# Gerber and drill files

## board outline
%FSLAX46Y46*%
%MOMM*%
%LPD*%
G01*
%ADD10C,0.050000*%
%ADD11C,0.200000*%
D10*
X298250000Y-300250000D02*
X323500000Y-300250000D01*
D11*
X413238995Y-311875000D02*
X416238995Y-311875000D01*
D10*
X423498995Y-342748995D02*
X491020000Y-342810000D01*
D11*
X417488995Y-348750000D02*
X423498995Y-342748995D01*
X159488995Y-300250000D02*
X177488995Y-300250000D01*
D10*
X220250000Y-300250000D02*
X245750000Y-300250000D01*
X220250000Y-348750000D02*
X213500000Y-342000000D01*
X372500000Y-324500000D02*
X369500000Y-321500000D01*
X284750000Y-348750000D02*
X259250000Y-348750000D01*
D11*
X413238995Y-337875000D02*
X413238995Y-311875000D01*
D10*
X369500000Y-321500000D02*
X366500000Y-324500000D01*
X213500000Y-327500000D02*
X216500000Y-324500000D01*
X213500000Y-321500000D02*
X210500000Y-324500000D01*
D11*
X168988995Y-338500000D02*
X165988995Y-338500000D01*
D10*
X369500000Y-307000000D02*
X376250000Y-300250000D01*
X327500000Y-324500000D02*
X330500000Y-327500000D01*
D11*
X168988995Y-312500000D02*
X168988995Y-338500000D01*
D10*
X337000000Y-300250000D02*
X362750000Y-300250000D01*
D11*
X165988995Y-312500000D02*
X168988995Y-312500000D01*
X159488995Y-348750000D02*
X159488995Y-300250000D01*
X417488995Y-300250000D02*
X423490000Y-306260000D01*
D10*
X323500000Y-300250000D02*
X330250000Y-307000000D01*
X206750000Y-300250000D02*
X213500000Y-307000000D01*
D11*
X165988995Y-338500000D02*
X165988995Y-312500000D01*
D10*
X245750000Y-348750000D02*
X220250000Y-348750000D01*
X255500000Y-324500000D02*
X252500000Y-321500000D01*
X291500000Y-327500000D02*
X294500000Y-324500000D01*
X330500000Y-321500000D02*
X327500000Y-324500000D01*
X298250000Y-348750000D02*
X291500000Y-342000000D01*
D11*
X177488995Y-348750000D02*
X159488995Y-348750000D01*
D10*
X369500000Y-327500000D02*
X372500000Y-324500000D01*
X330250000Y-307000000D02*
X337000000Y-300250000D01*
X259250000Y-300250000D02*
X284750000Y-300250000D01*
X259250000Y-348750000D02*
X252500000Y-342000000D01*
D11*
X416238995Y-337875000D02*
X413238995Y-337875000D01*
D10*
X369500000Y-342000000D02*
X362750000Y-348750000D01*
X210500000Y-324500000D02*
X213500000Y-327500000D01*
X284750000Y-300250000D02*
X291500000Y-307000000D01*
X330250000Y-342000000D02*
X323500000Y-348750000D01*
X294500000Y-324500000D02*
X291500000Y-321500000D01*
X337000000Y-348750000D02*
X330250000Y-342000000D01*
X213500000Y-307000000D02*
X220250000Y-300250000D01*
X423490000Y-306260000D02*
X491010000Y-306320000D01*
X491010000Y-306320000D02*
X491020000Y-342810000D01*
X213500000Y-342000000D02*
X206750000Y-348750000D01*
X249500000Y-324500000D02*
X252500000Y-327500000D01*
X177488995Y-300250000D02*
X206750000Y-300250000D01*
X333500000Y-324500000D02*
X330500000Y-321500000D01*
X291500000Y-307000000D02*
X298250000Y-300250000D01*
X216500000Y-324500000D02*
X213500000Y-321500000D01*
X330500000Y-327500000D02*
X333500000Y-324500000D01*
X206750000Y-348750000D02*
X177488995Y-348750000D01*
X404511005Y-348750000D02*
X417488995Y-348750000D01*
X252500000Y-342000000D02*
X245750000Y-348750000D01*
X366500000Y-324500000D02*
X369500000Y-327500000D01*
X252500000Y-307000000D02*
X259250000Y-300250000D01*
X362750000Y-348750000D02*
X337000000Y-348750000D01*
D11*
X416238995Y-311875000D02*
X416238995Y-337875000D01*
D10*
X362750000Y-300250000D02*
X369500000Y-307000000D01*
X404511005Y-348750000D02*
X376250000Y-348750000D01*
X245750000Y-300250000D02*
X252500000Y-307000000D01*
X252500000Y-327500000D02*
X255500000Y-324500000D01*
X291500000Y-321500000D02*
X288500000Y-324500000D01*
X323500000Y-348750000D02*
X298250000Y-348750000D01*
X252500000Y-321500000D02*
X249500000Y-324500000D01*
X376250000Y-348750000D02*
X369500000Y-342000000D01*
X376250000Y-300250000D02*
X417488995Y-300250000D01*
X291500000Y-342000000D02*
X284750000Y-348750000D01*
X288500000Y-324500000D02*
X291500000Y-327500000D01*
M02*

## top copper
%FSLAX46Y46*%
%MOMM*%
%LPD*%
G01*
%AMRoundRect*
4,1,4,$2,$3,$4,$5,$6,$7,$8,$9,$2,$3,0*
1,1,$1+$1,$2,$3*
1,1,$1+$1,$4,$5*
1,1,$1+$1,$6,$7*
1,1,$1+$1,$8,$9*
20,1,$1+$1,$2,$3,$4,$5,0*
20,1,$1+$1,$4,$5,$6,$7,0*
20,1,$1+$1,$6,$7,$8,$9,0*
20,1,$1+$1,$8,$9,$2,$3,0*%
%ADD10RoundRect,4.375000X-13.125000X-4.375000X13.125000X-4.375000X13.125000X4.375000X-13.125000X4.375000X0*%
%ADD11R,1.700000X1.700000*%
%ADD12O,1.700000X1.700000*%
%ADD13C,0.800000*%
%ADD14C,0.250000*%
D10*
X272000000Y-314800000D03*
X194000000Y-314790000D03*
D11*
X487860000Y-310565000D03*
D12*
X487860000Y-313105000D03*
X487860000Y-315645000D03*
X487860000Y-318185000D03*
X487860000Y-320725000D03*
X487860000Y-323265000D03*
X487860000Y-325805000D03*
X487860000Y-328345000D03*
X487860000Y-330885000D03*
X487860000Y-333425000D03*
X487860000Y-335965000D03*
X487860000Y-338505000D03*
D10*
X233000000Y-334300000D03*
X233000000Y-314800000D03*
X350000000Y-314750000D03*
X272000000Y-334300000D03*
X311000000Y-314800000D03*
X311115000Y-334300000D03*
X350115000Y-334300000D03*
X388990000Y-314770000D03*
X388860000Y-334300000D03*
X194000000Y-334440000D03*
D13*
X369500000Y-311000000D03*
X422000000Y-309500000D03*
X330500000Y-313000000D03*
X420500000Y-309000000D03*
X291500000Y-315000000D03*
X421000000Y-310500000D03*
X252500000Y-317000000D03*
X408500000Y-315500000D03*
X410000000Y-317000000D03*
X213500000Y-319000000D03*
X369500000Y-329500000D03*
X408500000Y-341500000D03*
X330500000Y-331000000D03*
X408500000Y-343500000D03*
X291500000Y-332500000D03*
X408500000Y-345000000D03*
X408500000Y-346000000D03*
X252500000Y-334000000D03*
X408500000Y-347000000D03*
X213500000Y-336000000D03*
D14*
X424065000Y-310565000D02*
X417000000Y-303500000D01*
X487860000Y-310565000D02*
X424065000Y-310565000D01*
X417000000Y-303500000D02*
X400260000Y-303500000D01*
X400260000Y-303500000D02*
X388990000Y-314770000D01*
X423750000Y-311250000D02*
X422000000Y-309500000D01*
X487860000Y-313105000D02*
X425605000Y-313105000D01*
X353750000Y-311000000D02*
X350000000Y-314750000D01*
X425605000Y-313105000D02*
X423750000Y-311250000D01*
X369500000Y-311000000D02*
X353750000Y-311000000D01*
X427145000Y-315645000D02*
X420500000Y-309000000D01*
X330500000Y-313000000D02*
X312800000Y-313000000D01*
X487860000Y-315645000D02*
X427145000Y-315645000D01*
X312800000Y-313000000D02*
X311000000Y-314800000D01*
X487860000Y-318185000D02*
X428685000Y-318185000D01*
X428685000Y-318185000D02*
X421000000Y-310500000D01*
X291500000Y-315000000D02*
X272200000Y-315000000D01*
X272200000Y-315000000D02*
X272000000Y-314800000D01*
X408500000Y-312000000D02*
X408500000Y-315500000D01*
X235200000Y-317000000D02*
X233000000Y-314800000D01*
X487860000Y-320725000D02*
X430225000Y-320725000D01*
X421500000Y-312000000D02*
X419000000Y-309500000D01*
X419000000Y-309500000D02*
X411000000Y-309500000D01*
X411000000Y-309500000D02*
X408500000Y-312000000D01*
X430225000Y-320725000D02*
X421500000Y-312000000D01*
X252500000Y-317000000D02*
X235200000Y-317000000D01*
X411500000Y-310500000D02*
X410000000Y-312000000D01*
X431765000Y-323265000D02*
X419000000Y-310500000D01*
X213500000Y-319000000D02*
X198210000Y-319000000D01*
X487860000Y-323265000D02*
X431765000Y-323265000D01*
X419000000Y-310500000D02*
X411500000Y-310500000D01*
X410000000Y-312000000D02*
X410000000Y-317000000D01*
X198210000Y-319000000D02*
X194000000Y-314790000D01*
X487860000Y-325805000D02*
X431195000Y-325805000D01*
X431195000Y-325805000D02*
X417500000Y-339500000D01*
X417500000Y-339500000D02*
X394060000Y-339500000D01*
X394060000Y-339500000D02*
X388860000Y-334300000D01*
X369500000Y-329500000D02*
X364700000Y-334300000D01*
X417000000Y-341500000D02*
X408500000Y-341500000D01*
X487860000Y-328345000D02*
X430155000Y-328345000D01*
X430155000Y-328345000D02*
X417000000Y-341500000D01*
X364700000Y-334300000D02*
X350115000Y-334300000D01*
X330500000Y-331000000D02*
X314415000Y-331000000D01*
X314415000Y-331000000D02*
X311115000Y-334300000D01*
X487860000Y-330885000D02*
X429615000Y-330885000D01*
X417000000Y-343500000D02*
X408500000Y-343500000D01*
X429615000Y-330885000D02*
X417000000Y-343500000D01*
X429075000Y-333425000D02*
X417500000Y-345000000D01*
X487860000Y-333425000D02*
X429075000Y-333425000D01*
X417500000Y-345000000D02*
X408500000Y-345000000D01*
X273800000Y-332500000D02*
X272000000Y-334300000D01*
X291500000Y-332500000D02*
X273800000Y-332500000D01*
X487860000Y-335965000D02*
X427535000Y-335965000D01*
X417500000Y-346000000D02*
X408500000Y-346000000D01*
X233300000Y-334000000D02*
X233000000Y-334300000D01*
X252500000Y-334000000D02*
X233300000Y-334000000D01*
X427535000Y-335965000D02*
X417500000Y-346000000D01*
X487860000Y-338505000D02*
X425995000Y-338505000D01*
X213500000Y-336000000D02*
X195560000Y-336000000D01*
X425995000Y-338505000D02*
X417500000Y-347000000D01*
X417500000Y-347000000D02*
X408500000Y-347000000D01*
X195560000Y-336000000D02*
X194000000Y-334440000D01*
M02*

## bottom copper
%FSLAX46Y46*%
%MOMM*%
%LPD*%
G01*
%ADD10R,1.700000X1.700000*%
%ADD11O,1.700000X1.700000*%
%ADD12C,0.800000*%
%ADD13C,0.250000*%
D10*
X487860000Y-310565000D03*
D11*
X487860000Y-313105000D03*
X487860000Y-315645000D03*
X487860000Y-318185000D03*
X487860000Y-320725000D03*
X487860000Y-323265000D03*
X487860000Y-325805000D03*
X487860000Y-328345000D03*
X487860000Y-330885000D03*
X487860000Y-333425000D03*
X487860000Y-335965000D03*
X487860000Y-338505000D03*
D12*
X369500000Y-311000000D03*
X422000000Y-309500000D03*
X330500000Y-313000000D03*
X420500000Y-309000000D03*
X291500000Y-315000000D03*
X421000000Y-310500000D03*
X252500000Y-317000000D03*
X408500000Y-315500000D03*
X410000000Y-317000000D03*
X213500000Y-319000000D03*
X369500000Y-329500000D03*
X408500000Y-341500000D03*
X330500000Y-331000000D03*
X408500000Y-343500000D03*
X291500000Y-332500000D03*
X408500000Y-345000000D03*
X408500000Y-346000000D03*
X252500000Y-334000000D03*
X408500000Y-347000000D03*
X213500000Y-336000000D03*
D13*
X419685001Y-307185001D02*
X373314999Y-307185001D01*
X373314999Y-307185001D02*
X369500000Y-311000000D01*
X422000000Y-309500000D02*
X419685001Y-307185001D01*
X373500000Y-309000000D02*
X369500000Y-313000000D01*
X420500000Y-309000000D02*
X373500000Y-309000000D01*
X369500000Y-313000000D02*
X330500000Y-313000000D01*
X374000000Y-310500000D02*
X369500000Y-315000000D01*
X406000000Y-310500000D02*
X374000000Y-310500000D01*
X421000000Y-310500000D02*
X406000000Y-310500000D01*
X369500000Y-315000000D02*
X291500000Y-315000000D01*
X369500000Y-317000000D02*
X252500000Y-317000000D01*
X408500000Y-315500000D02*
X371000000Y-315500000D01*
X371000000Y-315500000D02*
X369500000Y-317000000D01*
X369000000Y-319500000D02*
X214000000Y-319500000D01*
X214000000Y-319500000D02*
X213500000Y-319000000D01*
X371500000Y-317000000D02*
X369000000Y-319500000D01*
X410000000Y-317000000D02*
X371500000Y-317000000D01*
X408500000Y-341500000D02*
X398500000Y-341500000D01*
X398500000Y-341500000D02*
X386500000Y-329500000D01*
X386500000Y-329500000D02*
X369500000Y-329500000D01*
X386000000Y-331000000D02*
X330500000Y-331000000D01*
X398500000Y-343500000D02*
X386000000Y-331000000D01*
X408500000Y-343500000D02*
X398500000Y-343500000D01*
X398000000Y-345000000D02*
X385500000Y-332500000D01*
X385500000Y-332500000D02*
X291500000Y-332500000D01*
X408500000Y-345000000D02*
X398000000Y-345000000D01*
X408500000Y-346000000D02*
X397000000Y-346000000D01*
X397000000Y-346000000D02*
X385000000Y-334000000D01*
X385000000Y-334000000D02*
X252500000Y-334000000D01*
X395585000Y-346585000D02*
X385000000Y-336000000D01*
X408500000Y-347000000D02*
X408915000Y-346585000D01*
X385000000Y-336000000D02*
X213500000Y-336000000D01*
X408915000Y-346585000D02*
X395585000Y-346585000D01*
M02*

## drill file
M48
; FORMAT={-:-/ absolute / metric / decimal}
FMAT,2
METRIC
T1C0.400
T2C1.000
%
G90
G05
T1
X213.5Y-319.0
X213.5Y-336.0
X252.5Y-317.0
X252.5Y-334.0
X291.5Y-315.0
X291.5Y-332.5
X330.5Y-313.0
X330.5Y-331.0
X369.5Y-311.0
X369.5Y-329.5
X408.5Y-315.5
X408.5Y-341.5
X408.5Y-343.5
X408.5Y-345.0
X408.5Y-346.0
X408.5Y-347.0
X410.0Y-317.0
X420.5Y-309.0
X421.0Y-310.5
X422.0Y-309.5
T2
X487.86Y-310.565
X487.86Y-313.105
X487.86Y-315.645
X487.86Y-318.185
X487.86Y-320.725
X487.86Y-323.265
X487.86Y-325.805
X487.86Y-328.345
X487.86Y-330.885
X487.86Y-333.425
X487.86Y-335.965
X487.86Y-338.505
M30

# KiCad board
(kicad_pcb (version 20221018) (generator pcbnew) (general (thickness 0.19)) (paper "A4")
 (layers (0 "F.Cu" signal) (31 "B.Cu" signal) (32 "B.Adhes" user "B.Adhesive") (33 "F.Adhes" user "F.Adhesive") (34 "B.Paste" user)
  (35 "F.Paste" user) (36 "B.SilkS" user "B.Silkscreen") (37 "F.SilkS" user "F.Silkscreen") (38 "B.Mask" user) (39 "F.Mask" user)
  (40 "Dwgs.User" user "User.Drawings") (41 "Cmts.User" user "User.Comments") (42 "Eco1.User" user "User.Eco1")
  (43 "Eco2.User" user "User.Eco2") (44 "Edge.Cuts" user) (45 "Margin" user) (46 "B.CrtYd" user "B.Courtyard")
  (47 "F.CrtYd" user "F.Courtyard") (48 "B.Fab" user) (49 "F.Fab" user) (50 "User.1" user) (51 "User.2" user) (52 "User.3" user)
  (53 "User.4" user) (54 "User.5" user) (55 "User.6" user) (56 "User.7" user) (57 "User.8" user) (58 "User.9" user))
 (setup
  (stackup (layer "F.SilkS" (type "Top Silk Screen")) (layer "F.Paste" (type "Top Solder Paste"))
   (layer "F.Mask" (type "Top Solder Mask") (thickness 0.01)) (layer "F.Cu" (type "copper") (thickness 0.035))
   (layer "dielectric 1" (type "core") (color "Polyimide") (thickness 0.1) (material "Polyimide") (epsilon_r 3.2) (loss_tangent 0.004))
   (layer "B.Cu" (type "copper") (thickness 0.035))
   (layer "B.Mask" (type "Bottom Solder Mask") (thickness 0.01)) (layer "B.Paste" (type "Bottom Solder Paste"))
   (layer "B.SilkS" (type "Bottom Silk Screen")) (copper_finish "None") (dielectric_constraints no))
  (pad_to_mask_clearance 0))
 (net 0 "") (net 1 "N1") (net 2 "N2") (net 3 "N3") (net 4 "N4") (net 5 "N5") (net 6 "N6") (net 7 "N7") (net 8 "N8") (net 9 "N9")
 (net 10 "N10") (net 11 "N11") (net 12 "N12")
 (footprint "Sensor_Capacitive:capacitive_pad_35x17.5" (layer "F.Cu") (at 254.52 323.5)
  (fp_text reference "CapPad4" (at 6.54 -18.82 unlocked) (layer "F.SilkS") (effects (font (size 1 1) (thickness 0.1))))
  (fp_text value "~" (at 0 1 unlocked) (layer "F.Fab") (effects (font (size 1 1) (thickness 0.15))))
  (pad "1" smd roundrect (at 17.48 -8.7) (size 35 17.5) (layers "F.Cu" "F.Paste" "F.Mask") (roundrect_rratio 0.25) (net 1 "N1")))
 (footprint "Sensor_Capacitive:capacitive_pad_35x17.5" (layer "F.Cu") (at 176.52 323.49)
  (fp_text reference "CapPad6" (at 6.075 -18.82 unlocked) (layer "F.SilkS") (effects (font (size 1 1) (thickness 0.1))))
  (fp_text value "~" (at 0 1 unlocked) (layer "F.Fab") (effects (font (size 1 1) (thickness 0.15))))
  (pad "1" smd roundrect (at 17.48 -8.7) (size 35 17.5) (layers "F.Cu" "F.Paste" "F.Mask") (roundrect_rratio 0.25) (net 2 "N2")))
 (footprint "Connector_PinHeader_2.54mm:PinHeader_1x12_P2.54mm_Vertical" (layer "F.Cu") (at 487.86 310.565)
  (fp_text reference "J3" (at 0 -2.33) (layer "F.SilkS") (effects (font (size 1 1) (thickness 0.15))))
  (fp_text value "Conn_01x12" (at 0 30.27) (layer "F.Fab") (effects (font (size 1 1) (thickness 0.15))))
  (pad "1" thru_hole rect (at 0 0) (size 1.7 1.7) (drill 1) (layers "*.Cu" "*.Mask") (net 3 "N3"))
  (pad "2" thru_hole oval (at 0 2.54) (size 1.7 1.7) (drill 1) (layers "*.Cu" "*.Mask") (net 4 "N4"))
  (pad "3" thru_hole oval (at 0 5.08) (size 1.7 1.7) (drill 1) (layers "*.Cu" "*.Mask") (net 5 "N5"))
  (pad "4" thru_hole oval (at 0 7.62) (size 1.7 1.7) (drill 1) (layers "*.Cu" "*.Mask") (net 1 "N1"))
  (pad "5" thru_hole oval (at 0 10.16) (size 1.7 1.7) (drill 1) (layers "*.Cu" "*.Mask") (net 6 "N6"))
  (pad "6" thru_hole oval (at 0 12.7) (size 1.7 1.7) (drill 1) (layers "*.Cu" "*.Mask") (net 2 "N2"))
  (pad "7" thru_hole oval (at 0 15.24) (size 1.7 1.7) (drill 1) (layers "*.Cu" "*.Mask") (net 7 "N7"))
  (pad "8" thru_hole oval (at 0 17.78) (size 1.7 1.7) (drill 1) (layers "*.Cu" "*.Mask") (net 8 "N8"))
  (pad "9" thru_hole oval (at 0 20.32) (size 1.7 1.7) (drill 1) (layers "*.Cu" "*.Mask") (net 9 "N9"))
  (pad "10" thru_hole oval (at 0 22.86) (size 1.7 1.7) (drill 1) (layers "*.Cu" "*.Mask") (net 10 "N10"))
  (pad "11" thru_hole oval (at 0 25.4) (size 1.7 1.7) (drill 1) (layers "*.Cu" "*.Mask") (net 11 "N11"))
  (pad "12" thru_hole oval (at 0 27.94) (size 1.7 1.7) (drill 1) (layers "*.Cu" "*.Mask") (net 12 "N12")))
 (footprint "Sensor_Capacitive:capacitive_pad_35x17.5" (layer "F.Cu") (at 215.52 343)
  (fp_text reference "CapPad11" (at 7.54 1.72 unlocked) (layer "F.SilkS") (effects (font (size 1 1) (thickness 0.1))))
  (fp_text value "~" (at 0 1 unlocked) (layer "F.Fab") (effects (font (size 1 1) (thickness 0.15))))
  (pad "1" smd roundrect (at 17.48 -8.7) (size 35 17.5) (layers "F.Cu" "F.Paste" "F.Mask") (roundrect_rratio 0.25) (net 11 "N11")))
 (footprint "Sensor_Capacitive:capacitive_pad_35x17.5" (layer "F.Cu") (at 215.52 323.5)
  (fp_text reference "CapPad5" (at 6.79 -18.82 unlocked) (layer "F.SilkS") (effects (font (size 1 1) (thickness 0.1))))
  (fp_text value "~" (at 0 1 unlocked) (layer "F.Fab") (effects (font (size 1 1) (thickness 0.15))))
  (pad "1" smd roundrect (at 17.48 -8.7) (size 35 17.5) (layers "F.Cu" "F.Paste" "F.Mask") (roundrect_rratio 0.25) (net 6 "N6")))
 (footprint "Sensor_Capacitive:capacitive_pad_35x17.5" (layer "F.Cu") (at 332.52 323.45)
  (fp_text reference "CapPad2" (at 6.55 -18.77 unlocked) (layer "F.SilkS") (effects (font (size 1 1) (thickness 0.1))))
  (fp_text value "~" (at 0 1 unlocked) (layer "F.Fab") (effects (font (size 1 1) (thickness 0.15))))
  (pad "1" smd roundrect (at 17.48 -8.7) (size 35 17.5) (layers "F.Cu" "F.Paste" "F.Mask") (roundrect_rratio 0.25) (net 4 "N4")))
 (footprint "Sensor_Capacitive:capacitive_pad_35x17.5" (layer "F.Cu") (at 254.52 343)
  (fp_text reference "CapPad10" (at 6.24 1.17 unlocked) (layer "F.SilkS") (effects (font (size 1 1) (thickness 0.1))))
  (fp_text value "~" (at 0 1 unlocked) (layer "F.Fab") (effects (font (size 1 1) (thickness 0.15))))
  (pad "1" smd roundrect (at 17.48 -8.7) (size 35 17.5) (layers "F.Cu" "F.Paste" "F.Mask") (roundrect_rratio 0.25) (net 10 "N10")))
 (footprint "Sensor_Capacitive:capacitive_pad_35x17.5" (layer "F.Cu") (at 293.52 323.5)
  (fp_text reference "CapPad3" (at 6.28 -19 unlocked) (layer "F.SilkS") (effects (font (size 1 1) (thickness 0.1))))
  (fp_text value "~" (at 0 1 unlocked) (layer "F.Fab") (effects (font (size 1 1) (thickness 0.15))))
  (pad "1" smd roundrect (at 17.48 -8.7) (size 35 17.5) (layers "F.Cu" "F.Paste" "F.Mask") (roundrect_rratio 0.25) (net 5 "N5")))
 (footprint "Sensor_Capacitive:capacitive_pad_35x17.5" (layer "F.Cu") (at 293.635 343)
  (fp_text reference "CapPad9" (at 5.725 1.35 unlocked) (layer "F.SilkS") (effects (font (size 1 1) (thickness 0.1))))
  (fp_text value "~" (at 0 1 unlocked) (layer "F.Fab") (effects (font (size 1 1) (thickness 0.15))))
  (pad "1" smd roundrect (at 17.48 -8.7) (size 35 17.5) (layers "F.Cu" "F.Paste" "F.Mask") (roundrect_rratio 0.25) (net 9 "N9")))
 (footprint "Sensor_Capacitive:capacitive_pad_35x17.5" (layer "F.Cu") (at 332.635 343)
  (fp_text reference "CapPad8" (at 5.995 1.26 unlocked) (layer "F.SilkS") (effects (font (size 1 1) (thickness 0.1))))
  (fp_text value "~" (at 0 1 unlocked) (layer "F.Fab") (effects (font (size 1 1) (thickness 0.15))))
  (pad "1" smd roundrect (at 17.48 -8.7) (size 35 17.5) (layers "F.Cu" "F.Paste" "F.Mask") (roundrect_rratio 0.25) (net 8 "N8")))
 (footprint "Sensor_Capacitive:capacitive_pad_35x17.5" (layer "F.Cu") (at 371.51 323.47)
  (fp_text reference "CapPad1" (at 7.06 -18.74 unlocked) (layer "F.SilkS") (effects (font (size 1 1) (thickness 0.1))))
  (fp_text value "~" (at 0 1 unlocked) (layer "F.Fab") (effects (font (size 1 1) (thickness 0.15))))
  (pad "1" smd roundrect (at 17.48 -8.7) (size 35 17.5) (layers "F.Cu" "F.Paste" "F.Mask") (roundrect_rratio 0.25) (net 3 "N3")))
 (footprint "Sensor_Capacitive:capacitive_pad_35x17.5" (layer "F.Cu") (at 371.38 343)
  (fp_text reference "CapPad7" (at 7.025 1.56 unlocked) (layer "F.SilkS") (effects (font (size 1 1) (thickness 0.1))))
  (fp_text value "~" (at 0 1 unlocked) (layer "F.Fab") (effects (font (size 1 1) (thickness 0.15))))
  (pad "1" smd roundrect (at 17.48 -8.7) (size 35 17.5) (layers "F.Cu" "F.Paste" "F.Mask") (roundrect_rratio 0.25) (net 7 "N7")))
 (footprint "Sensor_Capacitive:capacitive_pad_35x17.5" (layer "F.Cu") (at 176.52 343.14)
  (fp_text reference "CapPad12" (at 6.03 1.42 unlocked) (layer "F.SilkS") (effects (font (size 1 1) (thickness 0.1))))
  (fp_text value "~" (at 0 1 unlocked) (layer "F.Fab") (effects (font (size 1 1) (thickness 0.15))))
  (pad "1" smd roundrect (at 17.48 -8.7) (size 35 17.5) (layers "F.Cu" "F.Paste" "F.Mask") (roundrect_rratio 0.25) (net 12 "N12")))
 (gr_line (start 298.25 300.25) (end 323.5 300.25) (stroke (width 0.05) (type default)) (layer "Edge.Cuts"))
 (gr_line (start 413.238995 311.875) (end 416.238995 311.875) (stroke (width 0.2) (type solid)) (layer "Edge.Cuts"))
 (gr_line (start 423.498995 342.748995) (end 491.02 342.81) (stroke (width 0.05) (type default)) (layer "Edge.Cuts"))
 (gr_line (start 417.488995 348.75) (end 423.498995 342.748995) (stroke (width 0.2) (type solid)) (layer "Edge.Cuts"))
 (gr_line (start 159.488995 300.25) (end 177.488995 300.25) (stroke (width 0.2) (type solid)) (layer "Edge.Cuts"))
 (gr_line (start 220.25 300.25) (end 245.75 300.25) (stroke (width 0.05) (type default)) (layer "Edge.Cuts"))
 (gr_line (start 220.25 348.75) (end 213.5 342) (stroke (width 0.05) (type default)) (layer "Edge.Cuts"))
 (gr_line (start 372.5 324.5) (end 369.5 321.5) (stroke (width 0.05) (type default)) (layer "Edge.Cuts"))
 (gr_line (start 284.75 348.75) (end 259.25 348.75) (stroke (width 0.05) (type default)) (layer "Edge.Cuts"))
 (gr_line (start 413.238995 337.875) (end 413.238995 311.875) (stroke (width 0.2) (type solid)) (layer "Edge.Cuts"))
 (gr_line (start 369.5 321.5) (end 366.5 324.5) (stroke (width 0.05) (type default)) (layer "Edge.Cuts"))
 (gr_line (start 213.5 327.5) (end 216.5 324.5) (stroke (width 0.05) (type default)) (layer "Edge.Cuts"))
 (gr_line (start 213.5 321.5) (end 210.5 324.5) (stroke (width 0.05) (type default)) (layer "Edge.Cuts"))
 (gr_line (start 168.988995 338.5) (end 165.988995 338.5) (stroke (width 0.2) (type solid)) (layer "Edge.Cuts"))
 (gr_line (start 369.5 307) (end 376.25 300.25) (stroke (width 0.05) (type default)) (layer "Edge.Cuts"))
 (gr_line (start 327.5 324.5) (end 330.5 327.5) (stroke (width 0.05) (type default)) (layer "Edge.Cuts"))
 (gr_line (start 168.988995 312.5) (end 168.988995 338.5) (stroke (width 0.2) (type solid)) (layer "Edge.Cuts"))
 (gr_line (start 337 300.25) (end 362.75 300.25) (stroke (width 0.05) (type default)) (layer "Edge.Cuts"))
 (gr_line (start 165.988995 312.5) (end 168.988995 312.5) (stroke (width 0.2) (type solid)) (layer "Edge.Cuts"))
 (gr_line (start 159.488995 348.75) (end 159.488995 300.25) (stroke (width 0.2) (type solid)) (layer "Edge.Cuts"))
 (gr_line (start 417.488995 300.25) (end 423.49 306.26) (stroke (width 0.2) (type solid)) (layer "Edge.Cuts"))
 (gr_line (start 323.5 300.25) (end 330.25 307) (stroke (width 0.05) (type default)) (layer "Edge.Cuts"))
 (gr_line (start 206.75 300.25) (end 213.5 307) (stroke (width 0.05) (type default)) (layer "Edge.Cuts"))
 (gr_line (start 165.988995 338.5) (end 165.988995 312.5) (stroke (width 0.2) (type solid)) (layer "Edge.Cuts"))
 (gr_line (start 245.75 348.75) (end 220.25 348.75) (stroke (width 0.05) (type default)) (layer "Edge.Cuts"))
 (gr_line (start 255.5 324.5) (end 252.5 321.5) (stroke (width 0.05) (type default)) (layer "Edge.Cuts"))
 (gr_line (start 291.5 327.5) (end 294.5 324.5) (stroke (width 0.05) (type default)) (layer "Edge.Cuts"))
 (gr_line (start 330.5 321.5) (end 327.5 324.5) (stroke (width 0.05) (type default)) (layer "Edge.Cuts"))
 (gr_line (start 298.25 348.75) (end 291.5 342) (stroke (width 0.05) (type default)) (layer "Edge.Cuts"))
 (gr_line (start 177.488995 348.75) (end 159.488995 348.75) (stroke (width 0.2) (type solid)) (layer "Edge.Cuts"))
 (gr_line (start 369.5 327.5) (end 372.5 324.5) (stroke (width 0.05) (type default)) (layer "Edge.Cuts"))
 (gr_line (start 330.25 307) (end 337 300.25) (stroke (width 0.05) (type default)) (layer "Edge.Cuts"))
 (gr_line (start 259.25 300.25) (end 284.75 300.25) (stroke (width 0.05) (type default)) (layer "Edge.Cuts"))
 (gr_line (start 259.25 348.75) (end 252.5 342) (stroke (width 0.05) (type default)) (layer "Edge.Cuts"))
 (gr_line (start 416.238995 337.875) (end 413.238995 337.875) (stroke (width 0.2) (type solid)) (layer "Edge.Cuts"))
 (gr_line (start 369.5 342) (end 362.75 348.75) (stroke (width 0.05) (type default)) (layer "Edge.Cuts"))
 (gr_line (start 210.5 324.5) (end 213.5 327.5) (stroke (width 0.05) (type default)) (layer "Edge.Cuts"))
 (gr_line (start 284.75 300.25) (end 291.5 307) (stroke (width 0.05) (type default)) (layer "Edge.Cuts"))
 (gr_line (start 330.25 342) (end 323.5 348.75) (stroke (width 0.05) (type default)) (layer "Edge.Cuts"))
 (gr_line (start 294.5 324.5) (end 291.5 321.5) (stroke (width 0.05) (type default)) (layer "Edge.Cuts"))
 (gr_line (start 337 348.75) (end 330.25 342) (stroke (width 0.05) (type default)) (layer "Edge.Cuts"))
 (gr_line (start 213.5 307) (end 220.25 300.25) (stroke (width 0.05) (type default)) (layer "Edge.Cuts"))
 (gr_line (start 423.49 306.26) (end 491.01 306.32) (stroke (width 0.05) (type default)) (layer "Edge.Cuts"))
 (gr_line (start 491.01 306.32) (end 491.02 342.81) (stroke (width 0.05) (type default)) (layer "Edge.Cuts"))
 (gr_line (start 213.5 342) (end 206.75 348.75) (stroke (width 0.05) (type default)) (layer "Edge.Cuts"))
 (gr_line (start 249.5 324.5) (end 252.5 327.5) (stroke (width 0.05) (type default)) (layer "Edge.Cuts"))
 (gr_line (start 177.488995 300.25) (end 206.75 300.25) (stroke (width 0.05) (type default)) (layer "Edge.Cuts"))
 (gr_line (start 333.5 324.5) (end 330.5 321.5) (stroke (width 0.05) (type default)) (layer "Edge.Cuts"))
 (gr_line (start 291.5 307) (end 298.25 300.25) (stroke (width 0.05) (type default)) (layer "Edge.Cuts"))
 (gr_line (start 216.5 324.5) (end 213.5 321.5) (stroke (width 0.05) (type default)) (layer "Edge.Cuts"))
 (gr_line (start 330.5 327.5) (end 333.5 324.5) (stroke (width 0.05) (type default)) (layer "Edge.Cuts"))
 (gr_line (start 206.75 348.75) (end 177.488995 348.75) (stroke (width 0.05) (type default)) (layer "Edge.Cuts"))
 (gr_line (start 404.511005 348.75) (end 417.488995 348.75) (stroke (width 0.05) (type default)) (layer "Edge.Cuts"))
 (gr_line (start 252.5 342) (end 245.75 348.75) (stroke (width 0.05) (type default)) (layer "Edge.Cuts"))
 (gr_line (start 366.5 324.5) (end 369.5 327.5) (stroke (width 0.05) (type default)) (layer "Edge.Cuts"))
 (gr_line (start 252.5 307) (end 259.25 300.25) (stroke (width 0.05) (type default)) (layer "Edge.Cuts"))
 (gr_line (start 362.75 348.75) (end 337 348.75) (stroke (width 0.05) (type default)) (layer "Edge.Cuts"))
 (gr_line (start 416.238995 311.875) (end 416.238995 337.875) (stroke (width 0.2) (type solid)) (layer "Edge.Cuts"))
 (gr_line (start 362.75 300.25) (end 369.5 307) (stroke (width 0.05) (type default)) (layer "Edge.Cuts"))
 (gr_line (start 404.511005 348.75) (end 376.25 348.75) (stroke (width 0.05) (type default)) (layer "Edge.Cuts"))
 (gr_line (start 245.75 300.25) (end 252.5 307) (stroke (width 0.05) (type default)) (layer "Edge.Cuts"))
 (gr_line (start 252.5 327.5) (end 255.5 324.5) (stroke (width 0.05) (type default)) (layer "Edge.Cuts"))
 (gr_line (start 291.5 321.5) (end 288.5 324.5) (stroke (width 0.05) (type default)) (layer "Edge.Cuts"))
 (gr_line (start 323.5 348.75) (end 298.25 348.75) (stroke (width 0.05) (type default)) (layer "Edge.Cuts"))
 (gr_line (start 252.5 321.5) (end 249.5 324.5) (stroke (width 0.05) (type default)) (layer "Edge.Cuts"))
 (gr_line (start 376.25 348.75) (end 369.5 342) (stroke (width 0.05) (type default)) (layer "Edge.Cuts"))
 (gr_line (start 376.25 300.25) (end 417.488995 300.25) (stroke (width 0.05) (type default)) (layer "Edge.Cuts"))
 (gr_line (start 291.5 342) (end 284.75 348.75) (stroke (width 0.05) (type default)) (layer "Edge.Cuts"))
 (gr_line (start 288.5 324.5) (end 291.5 327.5) (stroke (width 0.05) (type default)) (layer "Edge.Cuts"))
 (segment (start 424.065 310.565) (end 417 303.5) (width 0.25) (layer "F.Cu") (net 3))
 (segment (start 487.86 310.565) (end 424.065 310.565) (width 0.25) (layer "F.Cu") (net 3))
 (segment (start 417 303.5) (end 400.26 303.5) (width 0.25) (layer "F.Cu") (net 3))
 (segment (start 400.26 303.5) (end 388.99 314.77) (width 0.25) (layer "F.Cu") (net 3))
 (segment (start 423.75 311.25) (end 422 309.5) (width 0.25) (layer "F.Cu") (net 4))
 (segment (start 487.86 313.105) (end 425.605 313.105) (width 0.25) (layer "F.Cu") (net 4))
 (segment (start 353.75 311) (end 350 314.75) (width 0.25) (layer "F.Cu") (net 4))
 (segment (start 425.605 313.105) (end 423.75 311.25) (width 0.25) (layer "F.Cu") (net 4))
 (segment (start 369.5 311) (end 353.75 311) (width 0.25) (layer "F.Cu") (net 4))
 (via (at 369.5 311) (size 0.8) (drill 0.4) (layers "F.Cu" "B.Cu") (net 4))
 (via (at 422 309.5) (size 0.8) (drill 0.4) (layers "F.Cu" "B.Cu") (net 4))
 (segment (start 419.685001 307.185001) (end 373.314999 307.185001) (width 0.25) (layer "B.Cu") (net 4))
 (segment (start 373.314999 307.185001) (end 369.5 311) (width 0.25) (layer "B.Cu") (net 4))
 (segment (start 422 309.5) (end 419.685001 307.185001) (width 0.25) (layer "B.Cu") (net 4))
 (segment (start 427.145 315.645) (end 420.5 309) (width 0.25) (layer "F.Cu") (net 5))
 (segment (start 330.5 313) (end 312.8 313) (width 0.25) (layer "F.Cu") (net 5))
 (segment (start 487.86 315.645) (end 427.145 315.645) (width 0.25) (layer "F.Cu") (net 5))
 (segment (start 312.8 313) (end 311 314.8) (width 0.25) (layer "F.Cu") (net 5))
 (via (at 330.5 313) (size 0.8) (drill 0.4) (layers "F.Cu" "B.Cu") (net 5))
 (via (at 420.5 309) (size 0.8) (drill 0.4) (layers "F.Cu" "B.Cu") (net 5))
 (segment (start 373.5 309) (end 369.5 313) (width 0.25) (layer "B.Cu") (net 5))
 (segment (start 420.5 309) (end 373.5 309) (width 0.25) (layer "B.Cu") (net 5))
 (segment (start 369.5 313) (end 330.5 313) (width 0.25) (layer "B.Cu") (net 5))
 (segment (start 487.86 318.185) (end 428.685 318.185) (width 0.25) (layer "F.Cu") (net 1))
 (segment (start 428.685 318.185) (end 421 310.5) (width 0.25) (layer "F.Cu") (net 1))
 (segment (start 291.5 315) (end 272.2 315) (width 0.25) (layer "F.Cu") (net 1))
 (segment (start 272.2 315) (end 272 314.8) (width 0.25) (layer "F.Cu") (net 1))
 (via (at 291.5 315) (size 0.8) (drill 0.4) (layers "F.Cu" "B.Cu") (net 1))
 (via (at 421 310.5) (size 0.8) (drill 0.4) (layers "F.Cu" "B.Cu") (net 1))
 (segment (start 374 310.5) (end 369.5 315) (width 0.25) (layer "B.Cu") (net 1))
 (segment (start 406 310.5) (end 374 310.5) (width 0.25) (layer "B.Cu") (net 1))
 (segment (start 421 310.5) (end 406 310.5) (width 0.25) (layer "B.Cu") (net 1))
 (segment (start 369.5 315) (end 291.5 315) (width 0.25) (layer "B.Cu") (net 1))
 (segment (start 408.5 312) (end 408.5 315.5) (width 0.25) (layer "F.Cu") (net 6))
 (segment (start 235.2 317) (end 233 314.8) (width 0.25) (layer "F.Cu") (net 6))
 (segment (start 487.86 320.725) (end 430.225 320.725) (width 0.25) (layer "F.Cu") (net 6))
 (segment (start 421.5 312) (end 419 309.5) (width 0.25) (layer "F.Cu") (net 6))
 (segment (start 419 309.5) (end 411 309.5) (width 0.25) (layer "F.Cu") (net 6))
 (segment (start 411 309.5) (end 408.5 312) (width 0.25) (layer "F.Cu") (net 6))
 (segment (start 430.225 320.725) (end 421.5 312) (width 0.25) (layer "F.Cu") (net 6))
 (segment (start 252.5 317) (end 235.2 317) (width 0.25) (layer "F.Cu") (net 6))
 (via (at 252.5 317) (size 0.8) (drill 0.4) (layers "F.Cu" "B.Cu") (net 6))
 (via (at 408.5 315.5) (size 0.8) (drill 0.4) (layers "F.Cu" "B.Cu") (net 6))
 (segment (start 369.5 317) (end 252.5 317) (width 0.25) (layer "B.Cu") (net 6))
 (segment (start 408.5 315.5) (end 371 315.5) (width 0.25) (layer "B.Cu") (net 6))
 (segment (start 371 315.5) (end 369.5 317) (width 0.25) (layer "B.Cu") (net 6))
 (segment (start 411.5 310.5) (end 410 312) (width 0.25) (layer "F.Cu") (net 2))
 (segment (start 431.765 323.265) (end 419 310.5) (width 0.25) (layer "F.Cu") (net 2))
 (segment (start 213.5 319) (end 198.21 319) (width 0.25) (layer "F.Cu") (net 2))
 (segment (start 487.86 323.265) (end 431.765 323.265) (width 0.25) (layer "F.Cu") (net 2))
 (segment (start 419 310.5) (end 411.5 310.5) (width 0.25) (layer "F.Cu") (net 2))
 (segment (start 410 312) (end 410 317) (width 0.25) (layer "F.Cu") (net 2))
 (segment (start 198.21 319) (end 194 314.79) (width 0.25) (layer "F.Cu") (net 2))
 (via (at 410 317) (size 0.8) (drill 0.4) (layers "F.Cu" "B.Cu") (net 2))
 (via (at 213.5 319) (size 0.8) (drill 0.4) (layers "F.Cu" "B.Cu") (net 2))
 (segment (start 369 319.5) (end 214 319.5) (width 0.25) (layer "B.Cu") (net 2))
 (segment (start 214 319.5) (end 213.5 319) (width 0.25) (layer "B.Cu") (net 2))
 (segment (start 371.5 317) (end 369 319.5) (width 0.25) (layer "B.Cu") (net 2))
 (segment (start 410 317) (end 371.5 317) (width 0.25) (layer "B.Cu") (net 2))
 (segment (start 487.86 325.805) (end 431.195 325.805) (width 0.25) (layer "F.Cu") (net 7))
 (segment (start 431.195 325.805) (end 417.5 339.5) (width 0.25) (layer "F.Cu") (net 7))
 (segment (start 417.5 339.5) (end 394.06 339.5) (width 0.25) (layer "F.Cu") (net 7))
 (segment (start 394.06 339.5) (end 388.86 334.3) (width 0.25) (layer "F.Cu") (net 7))
 (segment (start 369.5 329.5) (end 364.7 334.3) (width 0.25) (layer "F.Cu") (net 8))
 (segment (start 417 341.5) (end 408.5 341.5) (width 0.25) (layer "F.Cu") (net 8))
 (segment (start 487.86 328.345) (end 430.155 328.345) (width 0.25) (layer "F.Cu") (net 8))
 (segment (start 430.155 328.345) (end 417 341.5) (width 0.25) (layer "F.Cu") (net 8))
 (segment (start 364.7 334.3) (end 350.115 334.3) (width 0.25) (layer "F.Cu") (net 8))
 (via (at 369.5 329.5) (size 0.8) (drill 0.4) (layers "F.Cu" "B.Cu") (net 8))
 (via (at 408.5 341.5) (size 0.8) (drill 0.4) (layers "F.Cu" "B.Cu") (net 8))
 (segment (start 408.5 341.5) (end 398.5 341.5) (width 0.25) (layer "B.Cu") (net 8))
 (segment (start 398.5 341.5) (end 386.5 329.5) (width 0.25) (layer "B.Cu") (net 8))
 (segment (start 386.5 329.5) (end 369.5 329.5) (width 0.25) (layer "B.Cu") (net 8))
 (segment (start 330.5 331) (end 314.415 331) (width 0.25) (layer "F.Cu") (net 9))
 (segment (start 314.415 331) (end 311.115 334.3) (width 0.25) (layer "F.Cu") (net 9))
 (segment (start 487.86 330.885) (end 429.615 330.885) (width 0.25) (layer "F.Cu") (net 9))
 (segment (start 417 343.5) (end 408.5 343.5) (width 0.25) (layer "F.Cu") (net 9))
 (segment (start 429.615 330.885) (end 417 343.5) (width 0.25) (layer "F.Cu") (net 9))
 (via (at 330.5 331) (size 0.8) (drill 0.4) (layers "F.Cu" "B.Cu") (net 9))
 (via (at 408.5 343.5) (size 0.8) (drill 0.4) (layers "F.Cu" "B.Cu") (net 9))
 (segment (start 386 331) (end 330.5 331) (width 0.25) (layer "B.Cu") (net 9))
 (segment (start 398.5 343.5) (end 386 331) (width 0.25) (layer "B.Cu") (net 9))
 (segment (start 408.5 343.5) (end 398.5 343.5) (width 0.25) (layer "B.Cu") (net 9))
 (segment (start 429.075 333.425) (end 417.5 345) (width 0.25) (layer "F.Cu") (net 10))
 (segment (start 487.86 333.425) (end 429.075 333.425) (width 0.25) (layer "F.Cu") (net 10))
 (segment (start 417.5 345) (end 408.5 345) (width 0.25) (layer "F.Cu") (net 10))
 (segment (start 273.8 332.5) (end 272 334.3) (width 0.25) (layer "F.Cu") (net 10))
 (segment (start 291.5 332.5) (end 273.8 332.5) (width 0.25) (layer "F.Cu") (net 10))
 (via (at 291.5 332.5) (size 0.8) (drill 0.4) (layers "F.Cu" "B.Cu") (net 10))
 (via (at 408.5 345) (size 0.8) (drill 0.4) (layers "F.Cu" "B.Cu") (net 10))
 (segment (start 398 345) (end 385.5 332.5) (width 0.25) (layer "B.Cu") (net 10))
 (segment (start 385.5 332.5) (end 291.5 332.5) (width 0.25) (layer "B.Cu") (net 10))
 (segment (start 408.5 345) (end 398 345) (width 0.25) (layer "B.Cu") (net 10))
 (segment (start 487.86 335.965) (end 427.535 335.965) (width 0.25) (layer "F.Cu") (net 11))
 (segment (start 417.5 346) (end 408.5 346) (width 0.25) (layer "F.Cu") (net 11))
 (segment (start 233.3 334) (end 233 334.3) (width 0.25) (layer "F.Cu") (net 11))
 (segment (start 252.5 334) (end 233.3 334) (width 0.25) (layer "F.Cu") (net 11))
 (segment (start 427.535 335.965) (end 417.5 346) (width 0.25) (layer "F.Cu") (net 11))
 (via (at 408.5 346) (size 0.8) (drill 0.4) (layers "F.Cu" "B.Cu") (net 11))
 (via (at 252.5 334) (size 0.8) (drill 0.4) (layers "F.Cu" "B.Cu") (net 11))
 (segment (start 408.5 346) (end 397 346) (width 0.25) (layer "B.Cu") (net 11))
 (segment (start 397 346) (end 385 334) (width 0.25) (layer "B.Cu") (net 11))
 (segment (start 385 334) (end 252.5 334) (width 0.25) (layer "B.Cu") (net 11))
 (segment (start 487.86 338.505) (end 425.995 338.505) (width 0.25) (layer "F.Cu") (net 12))
 (segment (start 213.5 336) (end 195.56 336) (width 0.25) (layer "F.Cu") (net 12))
 (segment (start 425.995 338.505) (end 417.5 347) (width 0.25) (layer "F.Cu") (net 12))
 (segment (start 417.5 347) (end 408.5 347) (width 0.25) (layer "F.Cu") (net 12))
 (segment (start 195.56 336) (end 194 334.44) (width 0.25) (layer "F.Cu") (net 12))
 (via (at 408.5 347) (size 0.8) (drill 0.4) (layers "F.Cu" "B.Cu") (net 12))
 (via (at 213.5 336) (size 0.8) (drill 0.4) (layers "F.Cu" "B.Cu") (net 12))
 (segment (start 395.585 346.585) (end 385 336) (width 0.25) (layer "B.Cu") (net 12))
 (segment (start 408.5 347) (end 408.915 346.585) (width 0.25) (layer "B.Cu") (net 12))
 (segment (start 385 336) (end 213.5 336) (width 0.25) (layer "B.Cu") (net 12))
 (segment (start 408.915 346.585) (end 395.585 346.585) (width 0.25) (layer "B.Cu") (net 12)))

